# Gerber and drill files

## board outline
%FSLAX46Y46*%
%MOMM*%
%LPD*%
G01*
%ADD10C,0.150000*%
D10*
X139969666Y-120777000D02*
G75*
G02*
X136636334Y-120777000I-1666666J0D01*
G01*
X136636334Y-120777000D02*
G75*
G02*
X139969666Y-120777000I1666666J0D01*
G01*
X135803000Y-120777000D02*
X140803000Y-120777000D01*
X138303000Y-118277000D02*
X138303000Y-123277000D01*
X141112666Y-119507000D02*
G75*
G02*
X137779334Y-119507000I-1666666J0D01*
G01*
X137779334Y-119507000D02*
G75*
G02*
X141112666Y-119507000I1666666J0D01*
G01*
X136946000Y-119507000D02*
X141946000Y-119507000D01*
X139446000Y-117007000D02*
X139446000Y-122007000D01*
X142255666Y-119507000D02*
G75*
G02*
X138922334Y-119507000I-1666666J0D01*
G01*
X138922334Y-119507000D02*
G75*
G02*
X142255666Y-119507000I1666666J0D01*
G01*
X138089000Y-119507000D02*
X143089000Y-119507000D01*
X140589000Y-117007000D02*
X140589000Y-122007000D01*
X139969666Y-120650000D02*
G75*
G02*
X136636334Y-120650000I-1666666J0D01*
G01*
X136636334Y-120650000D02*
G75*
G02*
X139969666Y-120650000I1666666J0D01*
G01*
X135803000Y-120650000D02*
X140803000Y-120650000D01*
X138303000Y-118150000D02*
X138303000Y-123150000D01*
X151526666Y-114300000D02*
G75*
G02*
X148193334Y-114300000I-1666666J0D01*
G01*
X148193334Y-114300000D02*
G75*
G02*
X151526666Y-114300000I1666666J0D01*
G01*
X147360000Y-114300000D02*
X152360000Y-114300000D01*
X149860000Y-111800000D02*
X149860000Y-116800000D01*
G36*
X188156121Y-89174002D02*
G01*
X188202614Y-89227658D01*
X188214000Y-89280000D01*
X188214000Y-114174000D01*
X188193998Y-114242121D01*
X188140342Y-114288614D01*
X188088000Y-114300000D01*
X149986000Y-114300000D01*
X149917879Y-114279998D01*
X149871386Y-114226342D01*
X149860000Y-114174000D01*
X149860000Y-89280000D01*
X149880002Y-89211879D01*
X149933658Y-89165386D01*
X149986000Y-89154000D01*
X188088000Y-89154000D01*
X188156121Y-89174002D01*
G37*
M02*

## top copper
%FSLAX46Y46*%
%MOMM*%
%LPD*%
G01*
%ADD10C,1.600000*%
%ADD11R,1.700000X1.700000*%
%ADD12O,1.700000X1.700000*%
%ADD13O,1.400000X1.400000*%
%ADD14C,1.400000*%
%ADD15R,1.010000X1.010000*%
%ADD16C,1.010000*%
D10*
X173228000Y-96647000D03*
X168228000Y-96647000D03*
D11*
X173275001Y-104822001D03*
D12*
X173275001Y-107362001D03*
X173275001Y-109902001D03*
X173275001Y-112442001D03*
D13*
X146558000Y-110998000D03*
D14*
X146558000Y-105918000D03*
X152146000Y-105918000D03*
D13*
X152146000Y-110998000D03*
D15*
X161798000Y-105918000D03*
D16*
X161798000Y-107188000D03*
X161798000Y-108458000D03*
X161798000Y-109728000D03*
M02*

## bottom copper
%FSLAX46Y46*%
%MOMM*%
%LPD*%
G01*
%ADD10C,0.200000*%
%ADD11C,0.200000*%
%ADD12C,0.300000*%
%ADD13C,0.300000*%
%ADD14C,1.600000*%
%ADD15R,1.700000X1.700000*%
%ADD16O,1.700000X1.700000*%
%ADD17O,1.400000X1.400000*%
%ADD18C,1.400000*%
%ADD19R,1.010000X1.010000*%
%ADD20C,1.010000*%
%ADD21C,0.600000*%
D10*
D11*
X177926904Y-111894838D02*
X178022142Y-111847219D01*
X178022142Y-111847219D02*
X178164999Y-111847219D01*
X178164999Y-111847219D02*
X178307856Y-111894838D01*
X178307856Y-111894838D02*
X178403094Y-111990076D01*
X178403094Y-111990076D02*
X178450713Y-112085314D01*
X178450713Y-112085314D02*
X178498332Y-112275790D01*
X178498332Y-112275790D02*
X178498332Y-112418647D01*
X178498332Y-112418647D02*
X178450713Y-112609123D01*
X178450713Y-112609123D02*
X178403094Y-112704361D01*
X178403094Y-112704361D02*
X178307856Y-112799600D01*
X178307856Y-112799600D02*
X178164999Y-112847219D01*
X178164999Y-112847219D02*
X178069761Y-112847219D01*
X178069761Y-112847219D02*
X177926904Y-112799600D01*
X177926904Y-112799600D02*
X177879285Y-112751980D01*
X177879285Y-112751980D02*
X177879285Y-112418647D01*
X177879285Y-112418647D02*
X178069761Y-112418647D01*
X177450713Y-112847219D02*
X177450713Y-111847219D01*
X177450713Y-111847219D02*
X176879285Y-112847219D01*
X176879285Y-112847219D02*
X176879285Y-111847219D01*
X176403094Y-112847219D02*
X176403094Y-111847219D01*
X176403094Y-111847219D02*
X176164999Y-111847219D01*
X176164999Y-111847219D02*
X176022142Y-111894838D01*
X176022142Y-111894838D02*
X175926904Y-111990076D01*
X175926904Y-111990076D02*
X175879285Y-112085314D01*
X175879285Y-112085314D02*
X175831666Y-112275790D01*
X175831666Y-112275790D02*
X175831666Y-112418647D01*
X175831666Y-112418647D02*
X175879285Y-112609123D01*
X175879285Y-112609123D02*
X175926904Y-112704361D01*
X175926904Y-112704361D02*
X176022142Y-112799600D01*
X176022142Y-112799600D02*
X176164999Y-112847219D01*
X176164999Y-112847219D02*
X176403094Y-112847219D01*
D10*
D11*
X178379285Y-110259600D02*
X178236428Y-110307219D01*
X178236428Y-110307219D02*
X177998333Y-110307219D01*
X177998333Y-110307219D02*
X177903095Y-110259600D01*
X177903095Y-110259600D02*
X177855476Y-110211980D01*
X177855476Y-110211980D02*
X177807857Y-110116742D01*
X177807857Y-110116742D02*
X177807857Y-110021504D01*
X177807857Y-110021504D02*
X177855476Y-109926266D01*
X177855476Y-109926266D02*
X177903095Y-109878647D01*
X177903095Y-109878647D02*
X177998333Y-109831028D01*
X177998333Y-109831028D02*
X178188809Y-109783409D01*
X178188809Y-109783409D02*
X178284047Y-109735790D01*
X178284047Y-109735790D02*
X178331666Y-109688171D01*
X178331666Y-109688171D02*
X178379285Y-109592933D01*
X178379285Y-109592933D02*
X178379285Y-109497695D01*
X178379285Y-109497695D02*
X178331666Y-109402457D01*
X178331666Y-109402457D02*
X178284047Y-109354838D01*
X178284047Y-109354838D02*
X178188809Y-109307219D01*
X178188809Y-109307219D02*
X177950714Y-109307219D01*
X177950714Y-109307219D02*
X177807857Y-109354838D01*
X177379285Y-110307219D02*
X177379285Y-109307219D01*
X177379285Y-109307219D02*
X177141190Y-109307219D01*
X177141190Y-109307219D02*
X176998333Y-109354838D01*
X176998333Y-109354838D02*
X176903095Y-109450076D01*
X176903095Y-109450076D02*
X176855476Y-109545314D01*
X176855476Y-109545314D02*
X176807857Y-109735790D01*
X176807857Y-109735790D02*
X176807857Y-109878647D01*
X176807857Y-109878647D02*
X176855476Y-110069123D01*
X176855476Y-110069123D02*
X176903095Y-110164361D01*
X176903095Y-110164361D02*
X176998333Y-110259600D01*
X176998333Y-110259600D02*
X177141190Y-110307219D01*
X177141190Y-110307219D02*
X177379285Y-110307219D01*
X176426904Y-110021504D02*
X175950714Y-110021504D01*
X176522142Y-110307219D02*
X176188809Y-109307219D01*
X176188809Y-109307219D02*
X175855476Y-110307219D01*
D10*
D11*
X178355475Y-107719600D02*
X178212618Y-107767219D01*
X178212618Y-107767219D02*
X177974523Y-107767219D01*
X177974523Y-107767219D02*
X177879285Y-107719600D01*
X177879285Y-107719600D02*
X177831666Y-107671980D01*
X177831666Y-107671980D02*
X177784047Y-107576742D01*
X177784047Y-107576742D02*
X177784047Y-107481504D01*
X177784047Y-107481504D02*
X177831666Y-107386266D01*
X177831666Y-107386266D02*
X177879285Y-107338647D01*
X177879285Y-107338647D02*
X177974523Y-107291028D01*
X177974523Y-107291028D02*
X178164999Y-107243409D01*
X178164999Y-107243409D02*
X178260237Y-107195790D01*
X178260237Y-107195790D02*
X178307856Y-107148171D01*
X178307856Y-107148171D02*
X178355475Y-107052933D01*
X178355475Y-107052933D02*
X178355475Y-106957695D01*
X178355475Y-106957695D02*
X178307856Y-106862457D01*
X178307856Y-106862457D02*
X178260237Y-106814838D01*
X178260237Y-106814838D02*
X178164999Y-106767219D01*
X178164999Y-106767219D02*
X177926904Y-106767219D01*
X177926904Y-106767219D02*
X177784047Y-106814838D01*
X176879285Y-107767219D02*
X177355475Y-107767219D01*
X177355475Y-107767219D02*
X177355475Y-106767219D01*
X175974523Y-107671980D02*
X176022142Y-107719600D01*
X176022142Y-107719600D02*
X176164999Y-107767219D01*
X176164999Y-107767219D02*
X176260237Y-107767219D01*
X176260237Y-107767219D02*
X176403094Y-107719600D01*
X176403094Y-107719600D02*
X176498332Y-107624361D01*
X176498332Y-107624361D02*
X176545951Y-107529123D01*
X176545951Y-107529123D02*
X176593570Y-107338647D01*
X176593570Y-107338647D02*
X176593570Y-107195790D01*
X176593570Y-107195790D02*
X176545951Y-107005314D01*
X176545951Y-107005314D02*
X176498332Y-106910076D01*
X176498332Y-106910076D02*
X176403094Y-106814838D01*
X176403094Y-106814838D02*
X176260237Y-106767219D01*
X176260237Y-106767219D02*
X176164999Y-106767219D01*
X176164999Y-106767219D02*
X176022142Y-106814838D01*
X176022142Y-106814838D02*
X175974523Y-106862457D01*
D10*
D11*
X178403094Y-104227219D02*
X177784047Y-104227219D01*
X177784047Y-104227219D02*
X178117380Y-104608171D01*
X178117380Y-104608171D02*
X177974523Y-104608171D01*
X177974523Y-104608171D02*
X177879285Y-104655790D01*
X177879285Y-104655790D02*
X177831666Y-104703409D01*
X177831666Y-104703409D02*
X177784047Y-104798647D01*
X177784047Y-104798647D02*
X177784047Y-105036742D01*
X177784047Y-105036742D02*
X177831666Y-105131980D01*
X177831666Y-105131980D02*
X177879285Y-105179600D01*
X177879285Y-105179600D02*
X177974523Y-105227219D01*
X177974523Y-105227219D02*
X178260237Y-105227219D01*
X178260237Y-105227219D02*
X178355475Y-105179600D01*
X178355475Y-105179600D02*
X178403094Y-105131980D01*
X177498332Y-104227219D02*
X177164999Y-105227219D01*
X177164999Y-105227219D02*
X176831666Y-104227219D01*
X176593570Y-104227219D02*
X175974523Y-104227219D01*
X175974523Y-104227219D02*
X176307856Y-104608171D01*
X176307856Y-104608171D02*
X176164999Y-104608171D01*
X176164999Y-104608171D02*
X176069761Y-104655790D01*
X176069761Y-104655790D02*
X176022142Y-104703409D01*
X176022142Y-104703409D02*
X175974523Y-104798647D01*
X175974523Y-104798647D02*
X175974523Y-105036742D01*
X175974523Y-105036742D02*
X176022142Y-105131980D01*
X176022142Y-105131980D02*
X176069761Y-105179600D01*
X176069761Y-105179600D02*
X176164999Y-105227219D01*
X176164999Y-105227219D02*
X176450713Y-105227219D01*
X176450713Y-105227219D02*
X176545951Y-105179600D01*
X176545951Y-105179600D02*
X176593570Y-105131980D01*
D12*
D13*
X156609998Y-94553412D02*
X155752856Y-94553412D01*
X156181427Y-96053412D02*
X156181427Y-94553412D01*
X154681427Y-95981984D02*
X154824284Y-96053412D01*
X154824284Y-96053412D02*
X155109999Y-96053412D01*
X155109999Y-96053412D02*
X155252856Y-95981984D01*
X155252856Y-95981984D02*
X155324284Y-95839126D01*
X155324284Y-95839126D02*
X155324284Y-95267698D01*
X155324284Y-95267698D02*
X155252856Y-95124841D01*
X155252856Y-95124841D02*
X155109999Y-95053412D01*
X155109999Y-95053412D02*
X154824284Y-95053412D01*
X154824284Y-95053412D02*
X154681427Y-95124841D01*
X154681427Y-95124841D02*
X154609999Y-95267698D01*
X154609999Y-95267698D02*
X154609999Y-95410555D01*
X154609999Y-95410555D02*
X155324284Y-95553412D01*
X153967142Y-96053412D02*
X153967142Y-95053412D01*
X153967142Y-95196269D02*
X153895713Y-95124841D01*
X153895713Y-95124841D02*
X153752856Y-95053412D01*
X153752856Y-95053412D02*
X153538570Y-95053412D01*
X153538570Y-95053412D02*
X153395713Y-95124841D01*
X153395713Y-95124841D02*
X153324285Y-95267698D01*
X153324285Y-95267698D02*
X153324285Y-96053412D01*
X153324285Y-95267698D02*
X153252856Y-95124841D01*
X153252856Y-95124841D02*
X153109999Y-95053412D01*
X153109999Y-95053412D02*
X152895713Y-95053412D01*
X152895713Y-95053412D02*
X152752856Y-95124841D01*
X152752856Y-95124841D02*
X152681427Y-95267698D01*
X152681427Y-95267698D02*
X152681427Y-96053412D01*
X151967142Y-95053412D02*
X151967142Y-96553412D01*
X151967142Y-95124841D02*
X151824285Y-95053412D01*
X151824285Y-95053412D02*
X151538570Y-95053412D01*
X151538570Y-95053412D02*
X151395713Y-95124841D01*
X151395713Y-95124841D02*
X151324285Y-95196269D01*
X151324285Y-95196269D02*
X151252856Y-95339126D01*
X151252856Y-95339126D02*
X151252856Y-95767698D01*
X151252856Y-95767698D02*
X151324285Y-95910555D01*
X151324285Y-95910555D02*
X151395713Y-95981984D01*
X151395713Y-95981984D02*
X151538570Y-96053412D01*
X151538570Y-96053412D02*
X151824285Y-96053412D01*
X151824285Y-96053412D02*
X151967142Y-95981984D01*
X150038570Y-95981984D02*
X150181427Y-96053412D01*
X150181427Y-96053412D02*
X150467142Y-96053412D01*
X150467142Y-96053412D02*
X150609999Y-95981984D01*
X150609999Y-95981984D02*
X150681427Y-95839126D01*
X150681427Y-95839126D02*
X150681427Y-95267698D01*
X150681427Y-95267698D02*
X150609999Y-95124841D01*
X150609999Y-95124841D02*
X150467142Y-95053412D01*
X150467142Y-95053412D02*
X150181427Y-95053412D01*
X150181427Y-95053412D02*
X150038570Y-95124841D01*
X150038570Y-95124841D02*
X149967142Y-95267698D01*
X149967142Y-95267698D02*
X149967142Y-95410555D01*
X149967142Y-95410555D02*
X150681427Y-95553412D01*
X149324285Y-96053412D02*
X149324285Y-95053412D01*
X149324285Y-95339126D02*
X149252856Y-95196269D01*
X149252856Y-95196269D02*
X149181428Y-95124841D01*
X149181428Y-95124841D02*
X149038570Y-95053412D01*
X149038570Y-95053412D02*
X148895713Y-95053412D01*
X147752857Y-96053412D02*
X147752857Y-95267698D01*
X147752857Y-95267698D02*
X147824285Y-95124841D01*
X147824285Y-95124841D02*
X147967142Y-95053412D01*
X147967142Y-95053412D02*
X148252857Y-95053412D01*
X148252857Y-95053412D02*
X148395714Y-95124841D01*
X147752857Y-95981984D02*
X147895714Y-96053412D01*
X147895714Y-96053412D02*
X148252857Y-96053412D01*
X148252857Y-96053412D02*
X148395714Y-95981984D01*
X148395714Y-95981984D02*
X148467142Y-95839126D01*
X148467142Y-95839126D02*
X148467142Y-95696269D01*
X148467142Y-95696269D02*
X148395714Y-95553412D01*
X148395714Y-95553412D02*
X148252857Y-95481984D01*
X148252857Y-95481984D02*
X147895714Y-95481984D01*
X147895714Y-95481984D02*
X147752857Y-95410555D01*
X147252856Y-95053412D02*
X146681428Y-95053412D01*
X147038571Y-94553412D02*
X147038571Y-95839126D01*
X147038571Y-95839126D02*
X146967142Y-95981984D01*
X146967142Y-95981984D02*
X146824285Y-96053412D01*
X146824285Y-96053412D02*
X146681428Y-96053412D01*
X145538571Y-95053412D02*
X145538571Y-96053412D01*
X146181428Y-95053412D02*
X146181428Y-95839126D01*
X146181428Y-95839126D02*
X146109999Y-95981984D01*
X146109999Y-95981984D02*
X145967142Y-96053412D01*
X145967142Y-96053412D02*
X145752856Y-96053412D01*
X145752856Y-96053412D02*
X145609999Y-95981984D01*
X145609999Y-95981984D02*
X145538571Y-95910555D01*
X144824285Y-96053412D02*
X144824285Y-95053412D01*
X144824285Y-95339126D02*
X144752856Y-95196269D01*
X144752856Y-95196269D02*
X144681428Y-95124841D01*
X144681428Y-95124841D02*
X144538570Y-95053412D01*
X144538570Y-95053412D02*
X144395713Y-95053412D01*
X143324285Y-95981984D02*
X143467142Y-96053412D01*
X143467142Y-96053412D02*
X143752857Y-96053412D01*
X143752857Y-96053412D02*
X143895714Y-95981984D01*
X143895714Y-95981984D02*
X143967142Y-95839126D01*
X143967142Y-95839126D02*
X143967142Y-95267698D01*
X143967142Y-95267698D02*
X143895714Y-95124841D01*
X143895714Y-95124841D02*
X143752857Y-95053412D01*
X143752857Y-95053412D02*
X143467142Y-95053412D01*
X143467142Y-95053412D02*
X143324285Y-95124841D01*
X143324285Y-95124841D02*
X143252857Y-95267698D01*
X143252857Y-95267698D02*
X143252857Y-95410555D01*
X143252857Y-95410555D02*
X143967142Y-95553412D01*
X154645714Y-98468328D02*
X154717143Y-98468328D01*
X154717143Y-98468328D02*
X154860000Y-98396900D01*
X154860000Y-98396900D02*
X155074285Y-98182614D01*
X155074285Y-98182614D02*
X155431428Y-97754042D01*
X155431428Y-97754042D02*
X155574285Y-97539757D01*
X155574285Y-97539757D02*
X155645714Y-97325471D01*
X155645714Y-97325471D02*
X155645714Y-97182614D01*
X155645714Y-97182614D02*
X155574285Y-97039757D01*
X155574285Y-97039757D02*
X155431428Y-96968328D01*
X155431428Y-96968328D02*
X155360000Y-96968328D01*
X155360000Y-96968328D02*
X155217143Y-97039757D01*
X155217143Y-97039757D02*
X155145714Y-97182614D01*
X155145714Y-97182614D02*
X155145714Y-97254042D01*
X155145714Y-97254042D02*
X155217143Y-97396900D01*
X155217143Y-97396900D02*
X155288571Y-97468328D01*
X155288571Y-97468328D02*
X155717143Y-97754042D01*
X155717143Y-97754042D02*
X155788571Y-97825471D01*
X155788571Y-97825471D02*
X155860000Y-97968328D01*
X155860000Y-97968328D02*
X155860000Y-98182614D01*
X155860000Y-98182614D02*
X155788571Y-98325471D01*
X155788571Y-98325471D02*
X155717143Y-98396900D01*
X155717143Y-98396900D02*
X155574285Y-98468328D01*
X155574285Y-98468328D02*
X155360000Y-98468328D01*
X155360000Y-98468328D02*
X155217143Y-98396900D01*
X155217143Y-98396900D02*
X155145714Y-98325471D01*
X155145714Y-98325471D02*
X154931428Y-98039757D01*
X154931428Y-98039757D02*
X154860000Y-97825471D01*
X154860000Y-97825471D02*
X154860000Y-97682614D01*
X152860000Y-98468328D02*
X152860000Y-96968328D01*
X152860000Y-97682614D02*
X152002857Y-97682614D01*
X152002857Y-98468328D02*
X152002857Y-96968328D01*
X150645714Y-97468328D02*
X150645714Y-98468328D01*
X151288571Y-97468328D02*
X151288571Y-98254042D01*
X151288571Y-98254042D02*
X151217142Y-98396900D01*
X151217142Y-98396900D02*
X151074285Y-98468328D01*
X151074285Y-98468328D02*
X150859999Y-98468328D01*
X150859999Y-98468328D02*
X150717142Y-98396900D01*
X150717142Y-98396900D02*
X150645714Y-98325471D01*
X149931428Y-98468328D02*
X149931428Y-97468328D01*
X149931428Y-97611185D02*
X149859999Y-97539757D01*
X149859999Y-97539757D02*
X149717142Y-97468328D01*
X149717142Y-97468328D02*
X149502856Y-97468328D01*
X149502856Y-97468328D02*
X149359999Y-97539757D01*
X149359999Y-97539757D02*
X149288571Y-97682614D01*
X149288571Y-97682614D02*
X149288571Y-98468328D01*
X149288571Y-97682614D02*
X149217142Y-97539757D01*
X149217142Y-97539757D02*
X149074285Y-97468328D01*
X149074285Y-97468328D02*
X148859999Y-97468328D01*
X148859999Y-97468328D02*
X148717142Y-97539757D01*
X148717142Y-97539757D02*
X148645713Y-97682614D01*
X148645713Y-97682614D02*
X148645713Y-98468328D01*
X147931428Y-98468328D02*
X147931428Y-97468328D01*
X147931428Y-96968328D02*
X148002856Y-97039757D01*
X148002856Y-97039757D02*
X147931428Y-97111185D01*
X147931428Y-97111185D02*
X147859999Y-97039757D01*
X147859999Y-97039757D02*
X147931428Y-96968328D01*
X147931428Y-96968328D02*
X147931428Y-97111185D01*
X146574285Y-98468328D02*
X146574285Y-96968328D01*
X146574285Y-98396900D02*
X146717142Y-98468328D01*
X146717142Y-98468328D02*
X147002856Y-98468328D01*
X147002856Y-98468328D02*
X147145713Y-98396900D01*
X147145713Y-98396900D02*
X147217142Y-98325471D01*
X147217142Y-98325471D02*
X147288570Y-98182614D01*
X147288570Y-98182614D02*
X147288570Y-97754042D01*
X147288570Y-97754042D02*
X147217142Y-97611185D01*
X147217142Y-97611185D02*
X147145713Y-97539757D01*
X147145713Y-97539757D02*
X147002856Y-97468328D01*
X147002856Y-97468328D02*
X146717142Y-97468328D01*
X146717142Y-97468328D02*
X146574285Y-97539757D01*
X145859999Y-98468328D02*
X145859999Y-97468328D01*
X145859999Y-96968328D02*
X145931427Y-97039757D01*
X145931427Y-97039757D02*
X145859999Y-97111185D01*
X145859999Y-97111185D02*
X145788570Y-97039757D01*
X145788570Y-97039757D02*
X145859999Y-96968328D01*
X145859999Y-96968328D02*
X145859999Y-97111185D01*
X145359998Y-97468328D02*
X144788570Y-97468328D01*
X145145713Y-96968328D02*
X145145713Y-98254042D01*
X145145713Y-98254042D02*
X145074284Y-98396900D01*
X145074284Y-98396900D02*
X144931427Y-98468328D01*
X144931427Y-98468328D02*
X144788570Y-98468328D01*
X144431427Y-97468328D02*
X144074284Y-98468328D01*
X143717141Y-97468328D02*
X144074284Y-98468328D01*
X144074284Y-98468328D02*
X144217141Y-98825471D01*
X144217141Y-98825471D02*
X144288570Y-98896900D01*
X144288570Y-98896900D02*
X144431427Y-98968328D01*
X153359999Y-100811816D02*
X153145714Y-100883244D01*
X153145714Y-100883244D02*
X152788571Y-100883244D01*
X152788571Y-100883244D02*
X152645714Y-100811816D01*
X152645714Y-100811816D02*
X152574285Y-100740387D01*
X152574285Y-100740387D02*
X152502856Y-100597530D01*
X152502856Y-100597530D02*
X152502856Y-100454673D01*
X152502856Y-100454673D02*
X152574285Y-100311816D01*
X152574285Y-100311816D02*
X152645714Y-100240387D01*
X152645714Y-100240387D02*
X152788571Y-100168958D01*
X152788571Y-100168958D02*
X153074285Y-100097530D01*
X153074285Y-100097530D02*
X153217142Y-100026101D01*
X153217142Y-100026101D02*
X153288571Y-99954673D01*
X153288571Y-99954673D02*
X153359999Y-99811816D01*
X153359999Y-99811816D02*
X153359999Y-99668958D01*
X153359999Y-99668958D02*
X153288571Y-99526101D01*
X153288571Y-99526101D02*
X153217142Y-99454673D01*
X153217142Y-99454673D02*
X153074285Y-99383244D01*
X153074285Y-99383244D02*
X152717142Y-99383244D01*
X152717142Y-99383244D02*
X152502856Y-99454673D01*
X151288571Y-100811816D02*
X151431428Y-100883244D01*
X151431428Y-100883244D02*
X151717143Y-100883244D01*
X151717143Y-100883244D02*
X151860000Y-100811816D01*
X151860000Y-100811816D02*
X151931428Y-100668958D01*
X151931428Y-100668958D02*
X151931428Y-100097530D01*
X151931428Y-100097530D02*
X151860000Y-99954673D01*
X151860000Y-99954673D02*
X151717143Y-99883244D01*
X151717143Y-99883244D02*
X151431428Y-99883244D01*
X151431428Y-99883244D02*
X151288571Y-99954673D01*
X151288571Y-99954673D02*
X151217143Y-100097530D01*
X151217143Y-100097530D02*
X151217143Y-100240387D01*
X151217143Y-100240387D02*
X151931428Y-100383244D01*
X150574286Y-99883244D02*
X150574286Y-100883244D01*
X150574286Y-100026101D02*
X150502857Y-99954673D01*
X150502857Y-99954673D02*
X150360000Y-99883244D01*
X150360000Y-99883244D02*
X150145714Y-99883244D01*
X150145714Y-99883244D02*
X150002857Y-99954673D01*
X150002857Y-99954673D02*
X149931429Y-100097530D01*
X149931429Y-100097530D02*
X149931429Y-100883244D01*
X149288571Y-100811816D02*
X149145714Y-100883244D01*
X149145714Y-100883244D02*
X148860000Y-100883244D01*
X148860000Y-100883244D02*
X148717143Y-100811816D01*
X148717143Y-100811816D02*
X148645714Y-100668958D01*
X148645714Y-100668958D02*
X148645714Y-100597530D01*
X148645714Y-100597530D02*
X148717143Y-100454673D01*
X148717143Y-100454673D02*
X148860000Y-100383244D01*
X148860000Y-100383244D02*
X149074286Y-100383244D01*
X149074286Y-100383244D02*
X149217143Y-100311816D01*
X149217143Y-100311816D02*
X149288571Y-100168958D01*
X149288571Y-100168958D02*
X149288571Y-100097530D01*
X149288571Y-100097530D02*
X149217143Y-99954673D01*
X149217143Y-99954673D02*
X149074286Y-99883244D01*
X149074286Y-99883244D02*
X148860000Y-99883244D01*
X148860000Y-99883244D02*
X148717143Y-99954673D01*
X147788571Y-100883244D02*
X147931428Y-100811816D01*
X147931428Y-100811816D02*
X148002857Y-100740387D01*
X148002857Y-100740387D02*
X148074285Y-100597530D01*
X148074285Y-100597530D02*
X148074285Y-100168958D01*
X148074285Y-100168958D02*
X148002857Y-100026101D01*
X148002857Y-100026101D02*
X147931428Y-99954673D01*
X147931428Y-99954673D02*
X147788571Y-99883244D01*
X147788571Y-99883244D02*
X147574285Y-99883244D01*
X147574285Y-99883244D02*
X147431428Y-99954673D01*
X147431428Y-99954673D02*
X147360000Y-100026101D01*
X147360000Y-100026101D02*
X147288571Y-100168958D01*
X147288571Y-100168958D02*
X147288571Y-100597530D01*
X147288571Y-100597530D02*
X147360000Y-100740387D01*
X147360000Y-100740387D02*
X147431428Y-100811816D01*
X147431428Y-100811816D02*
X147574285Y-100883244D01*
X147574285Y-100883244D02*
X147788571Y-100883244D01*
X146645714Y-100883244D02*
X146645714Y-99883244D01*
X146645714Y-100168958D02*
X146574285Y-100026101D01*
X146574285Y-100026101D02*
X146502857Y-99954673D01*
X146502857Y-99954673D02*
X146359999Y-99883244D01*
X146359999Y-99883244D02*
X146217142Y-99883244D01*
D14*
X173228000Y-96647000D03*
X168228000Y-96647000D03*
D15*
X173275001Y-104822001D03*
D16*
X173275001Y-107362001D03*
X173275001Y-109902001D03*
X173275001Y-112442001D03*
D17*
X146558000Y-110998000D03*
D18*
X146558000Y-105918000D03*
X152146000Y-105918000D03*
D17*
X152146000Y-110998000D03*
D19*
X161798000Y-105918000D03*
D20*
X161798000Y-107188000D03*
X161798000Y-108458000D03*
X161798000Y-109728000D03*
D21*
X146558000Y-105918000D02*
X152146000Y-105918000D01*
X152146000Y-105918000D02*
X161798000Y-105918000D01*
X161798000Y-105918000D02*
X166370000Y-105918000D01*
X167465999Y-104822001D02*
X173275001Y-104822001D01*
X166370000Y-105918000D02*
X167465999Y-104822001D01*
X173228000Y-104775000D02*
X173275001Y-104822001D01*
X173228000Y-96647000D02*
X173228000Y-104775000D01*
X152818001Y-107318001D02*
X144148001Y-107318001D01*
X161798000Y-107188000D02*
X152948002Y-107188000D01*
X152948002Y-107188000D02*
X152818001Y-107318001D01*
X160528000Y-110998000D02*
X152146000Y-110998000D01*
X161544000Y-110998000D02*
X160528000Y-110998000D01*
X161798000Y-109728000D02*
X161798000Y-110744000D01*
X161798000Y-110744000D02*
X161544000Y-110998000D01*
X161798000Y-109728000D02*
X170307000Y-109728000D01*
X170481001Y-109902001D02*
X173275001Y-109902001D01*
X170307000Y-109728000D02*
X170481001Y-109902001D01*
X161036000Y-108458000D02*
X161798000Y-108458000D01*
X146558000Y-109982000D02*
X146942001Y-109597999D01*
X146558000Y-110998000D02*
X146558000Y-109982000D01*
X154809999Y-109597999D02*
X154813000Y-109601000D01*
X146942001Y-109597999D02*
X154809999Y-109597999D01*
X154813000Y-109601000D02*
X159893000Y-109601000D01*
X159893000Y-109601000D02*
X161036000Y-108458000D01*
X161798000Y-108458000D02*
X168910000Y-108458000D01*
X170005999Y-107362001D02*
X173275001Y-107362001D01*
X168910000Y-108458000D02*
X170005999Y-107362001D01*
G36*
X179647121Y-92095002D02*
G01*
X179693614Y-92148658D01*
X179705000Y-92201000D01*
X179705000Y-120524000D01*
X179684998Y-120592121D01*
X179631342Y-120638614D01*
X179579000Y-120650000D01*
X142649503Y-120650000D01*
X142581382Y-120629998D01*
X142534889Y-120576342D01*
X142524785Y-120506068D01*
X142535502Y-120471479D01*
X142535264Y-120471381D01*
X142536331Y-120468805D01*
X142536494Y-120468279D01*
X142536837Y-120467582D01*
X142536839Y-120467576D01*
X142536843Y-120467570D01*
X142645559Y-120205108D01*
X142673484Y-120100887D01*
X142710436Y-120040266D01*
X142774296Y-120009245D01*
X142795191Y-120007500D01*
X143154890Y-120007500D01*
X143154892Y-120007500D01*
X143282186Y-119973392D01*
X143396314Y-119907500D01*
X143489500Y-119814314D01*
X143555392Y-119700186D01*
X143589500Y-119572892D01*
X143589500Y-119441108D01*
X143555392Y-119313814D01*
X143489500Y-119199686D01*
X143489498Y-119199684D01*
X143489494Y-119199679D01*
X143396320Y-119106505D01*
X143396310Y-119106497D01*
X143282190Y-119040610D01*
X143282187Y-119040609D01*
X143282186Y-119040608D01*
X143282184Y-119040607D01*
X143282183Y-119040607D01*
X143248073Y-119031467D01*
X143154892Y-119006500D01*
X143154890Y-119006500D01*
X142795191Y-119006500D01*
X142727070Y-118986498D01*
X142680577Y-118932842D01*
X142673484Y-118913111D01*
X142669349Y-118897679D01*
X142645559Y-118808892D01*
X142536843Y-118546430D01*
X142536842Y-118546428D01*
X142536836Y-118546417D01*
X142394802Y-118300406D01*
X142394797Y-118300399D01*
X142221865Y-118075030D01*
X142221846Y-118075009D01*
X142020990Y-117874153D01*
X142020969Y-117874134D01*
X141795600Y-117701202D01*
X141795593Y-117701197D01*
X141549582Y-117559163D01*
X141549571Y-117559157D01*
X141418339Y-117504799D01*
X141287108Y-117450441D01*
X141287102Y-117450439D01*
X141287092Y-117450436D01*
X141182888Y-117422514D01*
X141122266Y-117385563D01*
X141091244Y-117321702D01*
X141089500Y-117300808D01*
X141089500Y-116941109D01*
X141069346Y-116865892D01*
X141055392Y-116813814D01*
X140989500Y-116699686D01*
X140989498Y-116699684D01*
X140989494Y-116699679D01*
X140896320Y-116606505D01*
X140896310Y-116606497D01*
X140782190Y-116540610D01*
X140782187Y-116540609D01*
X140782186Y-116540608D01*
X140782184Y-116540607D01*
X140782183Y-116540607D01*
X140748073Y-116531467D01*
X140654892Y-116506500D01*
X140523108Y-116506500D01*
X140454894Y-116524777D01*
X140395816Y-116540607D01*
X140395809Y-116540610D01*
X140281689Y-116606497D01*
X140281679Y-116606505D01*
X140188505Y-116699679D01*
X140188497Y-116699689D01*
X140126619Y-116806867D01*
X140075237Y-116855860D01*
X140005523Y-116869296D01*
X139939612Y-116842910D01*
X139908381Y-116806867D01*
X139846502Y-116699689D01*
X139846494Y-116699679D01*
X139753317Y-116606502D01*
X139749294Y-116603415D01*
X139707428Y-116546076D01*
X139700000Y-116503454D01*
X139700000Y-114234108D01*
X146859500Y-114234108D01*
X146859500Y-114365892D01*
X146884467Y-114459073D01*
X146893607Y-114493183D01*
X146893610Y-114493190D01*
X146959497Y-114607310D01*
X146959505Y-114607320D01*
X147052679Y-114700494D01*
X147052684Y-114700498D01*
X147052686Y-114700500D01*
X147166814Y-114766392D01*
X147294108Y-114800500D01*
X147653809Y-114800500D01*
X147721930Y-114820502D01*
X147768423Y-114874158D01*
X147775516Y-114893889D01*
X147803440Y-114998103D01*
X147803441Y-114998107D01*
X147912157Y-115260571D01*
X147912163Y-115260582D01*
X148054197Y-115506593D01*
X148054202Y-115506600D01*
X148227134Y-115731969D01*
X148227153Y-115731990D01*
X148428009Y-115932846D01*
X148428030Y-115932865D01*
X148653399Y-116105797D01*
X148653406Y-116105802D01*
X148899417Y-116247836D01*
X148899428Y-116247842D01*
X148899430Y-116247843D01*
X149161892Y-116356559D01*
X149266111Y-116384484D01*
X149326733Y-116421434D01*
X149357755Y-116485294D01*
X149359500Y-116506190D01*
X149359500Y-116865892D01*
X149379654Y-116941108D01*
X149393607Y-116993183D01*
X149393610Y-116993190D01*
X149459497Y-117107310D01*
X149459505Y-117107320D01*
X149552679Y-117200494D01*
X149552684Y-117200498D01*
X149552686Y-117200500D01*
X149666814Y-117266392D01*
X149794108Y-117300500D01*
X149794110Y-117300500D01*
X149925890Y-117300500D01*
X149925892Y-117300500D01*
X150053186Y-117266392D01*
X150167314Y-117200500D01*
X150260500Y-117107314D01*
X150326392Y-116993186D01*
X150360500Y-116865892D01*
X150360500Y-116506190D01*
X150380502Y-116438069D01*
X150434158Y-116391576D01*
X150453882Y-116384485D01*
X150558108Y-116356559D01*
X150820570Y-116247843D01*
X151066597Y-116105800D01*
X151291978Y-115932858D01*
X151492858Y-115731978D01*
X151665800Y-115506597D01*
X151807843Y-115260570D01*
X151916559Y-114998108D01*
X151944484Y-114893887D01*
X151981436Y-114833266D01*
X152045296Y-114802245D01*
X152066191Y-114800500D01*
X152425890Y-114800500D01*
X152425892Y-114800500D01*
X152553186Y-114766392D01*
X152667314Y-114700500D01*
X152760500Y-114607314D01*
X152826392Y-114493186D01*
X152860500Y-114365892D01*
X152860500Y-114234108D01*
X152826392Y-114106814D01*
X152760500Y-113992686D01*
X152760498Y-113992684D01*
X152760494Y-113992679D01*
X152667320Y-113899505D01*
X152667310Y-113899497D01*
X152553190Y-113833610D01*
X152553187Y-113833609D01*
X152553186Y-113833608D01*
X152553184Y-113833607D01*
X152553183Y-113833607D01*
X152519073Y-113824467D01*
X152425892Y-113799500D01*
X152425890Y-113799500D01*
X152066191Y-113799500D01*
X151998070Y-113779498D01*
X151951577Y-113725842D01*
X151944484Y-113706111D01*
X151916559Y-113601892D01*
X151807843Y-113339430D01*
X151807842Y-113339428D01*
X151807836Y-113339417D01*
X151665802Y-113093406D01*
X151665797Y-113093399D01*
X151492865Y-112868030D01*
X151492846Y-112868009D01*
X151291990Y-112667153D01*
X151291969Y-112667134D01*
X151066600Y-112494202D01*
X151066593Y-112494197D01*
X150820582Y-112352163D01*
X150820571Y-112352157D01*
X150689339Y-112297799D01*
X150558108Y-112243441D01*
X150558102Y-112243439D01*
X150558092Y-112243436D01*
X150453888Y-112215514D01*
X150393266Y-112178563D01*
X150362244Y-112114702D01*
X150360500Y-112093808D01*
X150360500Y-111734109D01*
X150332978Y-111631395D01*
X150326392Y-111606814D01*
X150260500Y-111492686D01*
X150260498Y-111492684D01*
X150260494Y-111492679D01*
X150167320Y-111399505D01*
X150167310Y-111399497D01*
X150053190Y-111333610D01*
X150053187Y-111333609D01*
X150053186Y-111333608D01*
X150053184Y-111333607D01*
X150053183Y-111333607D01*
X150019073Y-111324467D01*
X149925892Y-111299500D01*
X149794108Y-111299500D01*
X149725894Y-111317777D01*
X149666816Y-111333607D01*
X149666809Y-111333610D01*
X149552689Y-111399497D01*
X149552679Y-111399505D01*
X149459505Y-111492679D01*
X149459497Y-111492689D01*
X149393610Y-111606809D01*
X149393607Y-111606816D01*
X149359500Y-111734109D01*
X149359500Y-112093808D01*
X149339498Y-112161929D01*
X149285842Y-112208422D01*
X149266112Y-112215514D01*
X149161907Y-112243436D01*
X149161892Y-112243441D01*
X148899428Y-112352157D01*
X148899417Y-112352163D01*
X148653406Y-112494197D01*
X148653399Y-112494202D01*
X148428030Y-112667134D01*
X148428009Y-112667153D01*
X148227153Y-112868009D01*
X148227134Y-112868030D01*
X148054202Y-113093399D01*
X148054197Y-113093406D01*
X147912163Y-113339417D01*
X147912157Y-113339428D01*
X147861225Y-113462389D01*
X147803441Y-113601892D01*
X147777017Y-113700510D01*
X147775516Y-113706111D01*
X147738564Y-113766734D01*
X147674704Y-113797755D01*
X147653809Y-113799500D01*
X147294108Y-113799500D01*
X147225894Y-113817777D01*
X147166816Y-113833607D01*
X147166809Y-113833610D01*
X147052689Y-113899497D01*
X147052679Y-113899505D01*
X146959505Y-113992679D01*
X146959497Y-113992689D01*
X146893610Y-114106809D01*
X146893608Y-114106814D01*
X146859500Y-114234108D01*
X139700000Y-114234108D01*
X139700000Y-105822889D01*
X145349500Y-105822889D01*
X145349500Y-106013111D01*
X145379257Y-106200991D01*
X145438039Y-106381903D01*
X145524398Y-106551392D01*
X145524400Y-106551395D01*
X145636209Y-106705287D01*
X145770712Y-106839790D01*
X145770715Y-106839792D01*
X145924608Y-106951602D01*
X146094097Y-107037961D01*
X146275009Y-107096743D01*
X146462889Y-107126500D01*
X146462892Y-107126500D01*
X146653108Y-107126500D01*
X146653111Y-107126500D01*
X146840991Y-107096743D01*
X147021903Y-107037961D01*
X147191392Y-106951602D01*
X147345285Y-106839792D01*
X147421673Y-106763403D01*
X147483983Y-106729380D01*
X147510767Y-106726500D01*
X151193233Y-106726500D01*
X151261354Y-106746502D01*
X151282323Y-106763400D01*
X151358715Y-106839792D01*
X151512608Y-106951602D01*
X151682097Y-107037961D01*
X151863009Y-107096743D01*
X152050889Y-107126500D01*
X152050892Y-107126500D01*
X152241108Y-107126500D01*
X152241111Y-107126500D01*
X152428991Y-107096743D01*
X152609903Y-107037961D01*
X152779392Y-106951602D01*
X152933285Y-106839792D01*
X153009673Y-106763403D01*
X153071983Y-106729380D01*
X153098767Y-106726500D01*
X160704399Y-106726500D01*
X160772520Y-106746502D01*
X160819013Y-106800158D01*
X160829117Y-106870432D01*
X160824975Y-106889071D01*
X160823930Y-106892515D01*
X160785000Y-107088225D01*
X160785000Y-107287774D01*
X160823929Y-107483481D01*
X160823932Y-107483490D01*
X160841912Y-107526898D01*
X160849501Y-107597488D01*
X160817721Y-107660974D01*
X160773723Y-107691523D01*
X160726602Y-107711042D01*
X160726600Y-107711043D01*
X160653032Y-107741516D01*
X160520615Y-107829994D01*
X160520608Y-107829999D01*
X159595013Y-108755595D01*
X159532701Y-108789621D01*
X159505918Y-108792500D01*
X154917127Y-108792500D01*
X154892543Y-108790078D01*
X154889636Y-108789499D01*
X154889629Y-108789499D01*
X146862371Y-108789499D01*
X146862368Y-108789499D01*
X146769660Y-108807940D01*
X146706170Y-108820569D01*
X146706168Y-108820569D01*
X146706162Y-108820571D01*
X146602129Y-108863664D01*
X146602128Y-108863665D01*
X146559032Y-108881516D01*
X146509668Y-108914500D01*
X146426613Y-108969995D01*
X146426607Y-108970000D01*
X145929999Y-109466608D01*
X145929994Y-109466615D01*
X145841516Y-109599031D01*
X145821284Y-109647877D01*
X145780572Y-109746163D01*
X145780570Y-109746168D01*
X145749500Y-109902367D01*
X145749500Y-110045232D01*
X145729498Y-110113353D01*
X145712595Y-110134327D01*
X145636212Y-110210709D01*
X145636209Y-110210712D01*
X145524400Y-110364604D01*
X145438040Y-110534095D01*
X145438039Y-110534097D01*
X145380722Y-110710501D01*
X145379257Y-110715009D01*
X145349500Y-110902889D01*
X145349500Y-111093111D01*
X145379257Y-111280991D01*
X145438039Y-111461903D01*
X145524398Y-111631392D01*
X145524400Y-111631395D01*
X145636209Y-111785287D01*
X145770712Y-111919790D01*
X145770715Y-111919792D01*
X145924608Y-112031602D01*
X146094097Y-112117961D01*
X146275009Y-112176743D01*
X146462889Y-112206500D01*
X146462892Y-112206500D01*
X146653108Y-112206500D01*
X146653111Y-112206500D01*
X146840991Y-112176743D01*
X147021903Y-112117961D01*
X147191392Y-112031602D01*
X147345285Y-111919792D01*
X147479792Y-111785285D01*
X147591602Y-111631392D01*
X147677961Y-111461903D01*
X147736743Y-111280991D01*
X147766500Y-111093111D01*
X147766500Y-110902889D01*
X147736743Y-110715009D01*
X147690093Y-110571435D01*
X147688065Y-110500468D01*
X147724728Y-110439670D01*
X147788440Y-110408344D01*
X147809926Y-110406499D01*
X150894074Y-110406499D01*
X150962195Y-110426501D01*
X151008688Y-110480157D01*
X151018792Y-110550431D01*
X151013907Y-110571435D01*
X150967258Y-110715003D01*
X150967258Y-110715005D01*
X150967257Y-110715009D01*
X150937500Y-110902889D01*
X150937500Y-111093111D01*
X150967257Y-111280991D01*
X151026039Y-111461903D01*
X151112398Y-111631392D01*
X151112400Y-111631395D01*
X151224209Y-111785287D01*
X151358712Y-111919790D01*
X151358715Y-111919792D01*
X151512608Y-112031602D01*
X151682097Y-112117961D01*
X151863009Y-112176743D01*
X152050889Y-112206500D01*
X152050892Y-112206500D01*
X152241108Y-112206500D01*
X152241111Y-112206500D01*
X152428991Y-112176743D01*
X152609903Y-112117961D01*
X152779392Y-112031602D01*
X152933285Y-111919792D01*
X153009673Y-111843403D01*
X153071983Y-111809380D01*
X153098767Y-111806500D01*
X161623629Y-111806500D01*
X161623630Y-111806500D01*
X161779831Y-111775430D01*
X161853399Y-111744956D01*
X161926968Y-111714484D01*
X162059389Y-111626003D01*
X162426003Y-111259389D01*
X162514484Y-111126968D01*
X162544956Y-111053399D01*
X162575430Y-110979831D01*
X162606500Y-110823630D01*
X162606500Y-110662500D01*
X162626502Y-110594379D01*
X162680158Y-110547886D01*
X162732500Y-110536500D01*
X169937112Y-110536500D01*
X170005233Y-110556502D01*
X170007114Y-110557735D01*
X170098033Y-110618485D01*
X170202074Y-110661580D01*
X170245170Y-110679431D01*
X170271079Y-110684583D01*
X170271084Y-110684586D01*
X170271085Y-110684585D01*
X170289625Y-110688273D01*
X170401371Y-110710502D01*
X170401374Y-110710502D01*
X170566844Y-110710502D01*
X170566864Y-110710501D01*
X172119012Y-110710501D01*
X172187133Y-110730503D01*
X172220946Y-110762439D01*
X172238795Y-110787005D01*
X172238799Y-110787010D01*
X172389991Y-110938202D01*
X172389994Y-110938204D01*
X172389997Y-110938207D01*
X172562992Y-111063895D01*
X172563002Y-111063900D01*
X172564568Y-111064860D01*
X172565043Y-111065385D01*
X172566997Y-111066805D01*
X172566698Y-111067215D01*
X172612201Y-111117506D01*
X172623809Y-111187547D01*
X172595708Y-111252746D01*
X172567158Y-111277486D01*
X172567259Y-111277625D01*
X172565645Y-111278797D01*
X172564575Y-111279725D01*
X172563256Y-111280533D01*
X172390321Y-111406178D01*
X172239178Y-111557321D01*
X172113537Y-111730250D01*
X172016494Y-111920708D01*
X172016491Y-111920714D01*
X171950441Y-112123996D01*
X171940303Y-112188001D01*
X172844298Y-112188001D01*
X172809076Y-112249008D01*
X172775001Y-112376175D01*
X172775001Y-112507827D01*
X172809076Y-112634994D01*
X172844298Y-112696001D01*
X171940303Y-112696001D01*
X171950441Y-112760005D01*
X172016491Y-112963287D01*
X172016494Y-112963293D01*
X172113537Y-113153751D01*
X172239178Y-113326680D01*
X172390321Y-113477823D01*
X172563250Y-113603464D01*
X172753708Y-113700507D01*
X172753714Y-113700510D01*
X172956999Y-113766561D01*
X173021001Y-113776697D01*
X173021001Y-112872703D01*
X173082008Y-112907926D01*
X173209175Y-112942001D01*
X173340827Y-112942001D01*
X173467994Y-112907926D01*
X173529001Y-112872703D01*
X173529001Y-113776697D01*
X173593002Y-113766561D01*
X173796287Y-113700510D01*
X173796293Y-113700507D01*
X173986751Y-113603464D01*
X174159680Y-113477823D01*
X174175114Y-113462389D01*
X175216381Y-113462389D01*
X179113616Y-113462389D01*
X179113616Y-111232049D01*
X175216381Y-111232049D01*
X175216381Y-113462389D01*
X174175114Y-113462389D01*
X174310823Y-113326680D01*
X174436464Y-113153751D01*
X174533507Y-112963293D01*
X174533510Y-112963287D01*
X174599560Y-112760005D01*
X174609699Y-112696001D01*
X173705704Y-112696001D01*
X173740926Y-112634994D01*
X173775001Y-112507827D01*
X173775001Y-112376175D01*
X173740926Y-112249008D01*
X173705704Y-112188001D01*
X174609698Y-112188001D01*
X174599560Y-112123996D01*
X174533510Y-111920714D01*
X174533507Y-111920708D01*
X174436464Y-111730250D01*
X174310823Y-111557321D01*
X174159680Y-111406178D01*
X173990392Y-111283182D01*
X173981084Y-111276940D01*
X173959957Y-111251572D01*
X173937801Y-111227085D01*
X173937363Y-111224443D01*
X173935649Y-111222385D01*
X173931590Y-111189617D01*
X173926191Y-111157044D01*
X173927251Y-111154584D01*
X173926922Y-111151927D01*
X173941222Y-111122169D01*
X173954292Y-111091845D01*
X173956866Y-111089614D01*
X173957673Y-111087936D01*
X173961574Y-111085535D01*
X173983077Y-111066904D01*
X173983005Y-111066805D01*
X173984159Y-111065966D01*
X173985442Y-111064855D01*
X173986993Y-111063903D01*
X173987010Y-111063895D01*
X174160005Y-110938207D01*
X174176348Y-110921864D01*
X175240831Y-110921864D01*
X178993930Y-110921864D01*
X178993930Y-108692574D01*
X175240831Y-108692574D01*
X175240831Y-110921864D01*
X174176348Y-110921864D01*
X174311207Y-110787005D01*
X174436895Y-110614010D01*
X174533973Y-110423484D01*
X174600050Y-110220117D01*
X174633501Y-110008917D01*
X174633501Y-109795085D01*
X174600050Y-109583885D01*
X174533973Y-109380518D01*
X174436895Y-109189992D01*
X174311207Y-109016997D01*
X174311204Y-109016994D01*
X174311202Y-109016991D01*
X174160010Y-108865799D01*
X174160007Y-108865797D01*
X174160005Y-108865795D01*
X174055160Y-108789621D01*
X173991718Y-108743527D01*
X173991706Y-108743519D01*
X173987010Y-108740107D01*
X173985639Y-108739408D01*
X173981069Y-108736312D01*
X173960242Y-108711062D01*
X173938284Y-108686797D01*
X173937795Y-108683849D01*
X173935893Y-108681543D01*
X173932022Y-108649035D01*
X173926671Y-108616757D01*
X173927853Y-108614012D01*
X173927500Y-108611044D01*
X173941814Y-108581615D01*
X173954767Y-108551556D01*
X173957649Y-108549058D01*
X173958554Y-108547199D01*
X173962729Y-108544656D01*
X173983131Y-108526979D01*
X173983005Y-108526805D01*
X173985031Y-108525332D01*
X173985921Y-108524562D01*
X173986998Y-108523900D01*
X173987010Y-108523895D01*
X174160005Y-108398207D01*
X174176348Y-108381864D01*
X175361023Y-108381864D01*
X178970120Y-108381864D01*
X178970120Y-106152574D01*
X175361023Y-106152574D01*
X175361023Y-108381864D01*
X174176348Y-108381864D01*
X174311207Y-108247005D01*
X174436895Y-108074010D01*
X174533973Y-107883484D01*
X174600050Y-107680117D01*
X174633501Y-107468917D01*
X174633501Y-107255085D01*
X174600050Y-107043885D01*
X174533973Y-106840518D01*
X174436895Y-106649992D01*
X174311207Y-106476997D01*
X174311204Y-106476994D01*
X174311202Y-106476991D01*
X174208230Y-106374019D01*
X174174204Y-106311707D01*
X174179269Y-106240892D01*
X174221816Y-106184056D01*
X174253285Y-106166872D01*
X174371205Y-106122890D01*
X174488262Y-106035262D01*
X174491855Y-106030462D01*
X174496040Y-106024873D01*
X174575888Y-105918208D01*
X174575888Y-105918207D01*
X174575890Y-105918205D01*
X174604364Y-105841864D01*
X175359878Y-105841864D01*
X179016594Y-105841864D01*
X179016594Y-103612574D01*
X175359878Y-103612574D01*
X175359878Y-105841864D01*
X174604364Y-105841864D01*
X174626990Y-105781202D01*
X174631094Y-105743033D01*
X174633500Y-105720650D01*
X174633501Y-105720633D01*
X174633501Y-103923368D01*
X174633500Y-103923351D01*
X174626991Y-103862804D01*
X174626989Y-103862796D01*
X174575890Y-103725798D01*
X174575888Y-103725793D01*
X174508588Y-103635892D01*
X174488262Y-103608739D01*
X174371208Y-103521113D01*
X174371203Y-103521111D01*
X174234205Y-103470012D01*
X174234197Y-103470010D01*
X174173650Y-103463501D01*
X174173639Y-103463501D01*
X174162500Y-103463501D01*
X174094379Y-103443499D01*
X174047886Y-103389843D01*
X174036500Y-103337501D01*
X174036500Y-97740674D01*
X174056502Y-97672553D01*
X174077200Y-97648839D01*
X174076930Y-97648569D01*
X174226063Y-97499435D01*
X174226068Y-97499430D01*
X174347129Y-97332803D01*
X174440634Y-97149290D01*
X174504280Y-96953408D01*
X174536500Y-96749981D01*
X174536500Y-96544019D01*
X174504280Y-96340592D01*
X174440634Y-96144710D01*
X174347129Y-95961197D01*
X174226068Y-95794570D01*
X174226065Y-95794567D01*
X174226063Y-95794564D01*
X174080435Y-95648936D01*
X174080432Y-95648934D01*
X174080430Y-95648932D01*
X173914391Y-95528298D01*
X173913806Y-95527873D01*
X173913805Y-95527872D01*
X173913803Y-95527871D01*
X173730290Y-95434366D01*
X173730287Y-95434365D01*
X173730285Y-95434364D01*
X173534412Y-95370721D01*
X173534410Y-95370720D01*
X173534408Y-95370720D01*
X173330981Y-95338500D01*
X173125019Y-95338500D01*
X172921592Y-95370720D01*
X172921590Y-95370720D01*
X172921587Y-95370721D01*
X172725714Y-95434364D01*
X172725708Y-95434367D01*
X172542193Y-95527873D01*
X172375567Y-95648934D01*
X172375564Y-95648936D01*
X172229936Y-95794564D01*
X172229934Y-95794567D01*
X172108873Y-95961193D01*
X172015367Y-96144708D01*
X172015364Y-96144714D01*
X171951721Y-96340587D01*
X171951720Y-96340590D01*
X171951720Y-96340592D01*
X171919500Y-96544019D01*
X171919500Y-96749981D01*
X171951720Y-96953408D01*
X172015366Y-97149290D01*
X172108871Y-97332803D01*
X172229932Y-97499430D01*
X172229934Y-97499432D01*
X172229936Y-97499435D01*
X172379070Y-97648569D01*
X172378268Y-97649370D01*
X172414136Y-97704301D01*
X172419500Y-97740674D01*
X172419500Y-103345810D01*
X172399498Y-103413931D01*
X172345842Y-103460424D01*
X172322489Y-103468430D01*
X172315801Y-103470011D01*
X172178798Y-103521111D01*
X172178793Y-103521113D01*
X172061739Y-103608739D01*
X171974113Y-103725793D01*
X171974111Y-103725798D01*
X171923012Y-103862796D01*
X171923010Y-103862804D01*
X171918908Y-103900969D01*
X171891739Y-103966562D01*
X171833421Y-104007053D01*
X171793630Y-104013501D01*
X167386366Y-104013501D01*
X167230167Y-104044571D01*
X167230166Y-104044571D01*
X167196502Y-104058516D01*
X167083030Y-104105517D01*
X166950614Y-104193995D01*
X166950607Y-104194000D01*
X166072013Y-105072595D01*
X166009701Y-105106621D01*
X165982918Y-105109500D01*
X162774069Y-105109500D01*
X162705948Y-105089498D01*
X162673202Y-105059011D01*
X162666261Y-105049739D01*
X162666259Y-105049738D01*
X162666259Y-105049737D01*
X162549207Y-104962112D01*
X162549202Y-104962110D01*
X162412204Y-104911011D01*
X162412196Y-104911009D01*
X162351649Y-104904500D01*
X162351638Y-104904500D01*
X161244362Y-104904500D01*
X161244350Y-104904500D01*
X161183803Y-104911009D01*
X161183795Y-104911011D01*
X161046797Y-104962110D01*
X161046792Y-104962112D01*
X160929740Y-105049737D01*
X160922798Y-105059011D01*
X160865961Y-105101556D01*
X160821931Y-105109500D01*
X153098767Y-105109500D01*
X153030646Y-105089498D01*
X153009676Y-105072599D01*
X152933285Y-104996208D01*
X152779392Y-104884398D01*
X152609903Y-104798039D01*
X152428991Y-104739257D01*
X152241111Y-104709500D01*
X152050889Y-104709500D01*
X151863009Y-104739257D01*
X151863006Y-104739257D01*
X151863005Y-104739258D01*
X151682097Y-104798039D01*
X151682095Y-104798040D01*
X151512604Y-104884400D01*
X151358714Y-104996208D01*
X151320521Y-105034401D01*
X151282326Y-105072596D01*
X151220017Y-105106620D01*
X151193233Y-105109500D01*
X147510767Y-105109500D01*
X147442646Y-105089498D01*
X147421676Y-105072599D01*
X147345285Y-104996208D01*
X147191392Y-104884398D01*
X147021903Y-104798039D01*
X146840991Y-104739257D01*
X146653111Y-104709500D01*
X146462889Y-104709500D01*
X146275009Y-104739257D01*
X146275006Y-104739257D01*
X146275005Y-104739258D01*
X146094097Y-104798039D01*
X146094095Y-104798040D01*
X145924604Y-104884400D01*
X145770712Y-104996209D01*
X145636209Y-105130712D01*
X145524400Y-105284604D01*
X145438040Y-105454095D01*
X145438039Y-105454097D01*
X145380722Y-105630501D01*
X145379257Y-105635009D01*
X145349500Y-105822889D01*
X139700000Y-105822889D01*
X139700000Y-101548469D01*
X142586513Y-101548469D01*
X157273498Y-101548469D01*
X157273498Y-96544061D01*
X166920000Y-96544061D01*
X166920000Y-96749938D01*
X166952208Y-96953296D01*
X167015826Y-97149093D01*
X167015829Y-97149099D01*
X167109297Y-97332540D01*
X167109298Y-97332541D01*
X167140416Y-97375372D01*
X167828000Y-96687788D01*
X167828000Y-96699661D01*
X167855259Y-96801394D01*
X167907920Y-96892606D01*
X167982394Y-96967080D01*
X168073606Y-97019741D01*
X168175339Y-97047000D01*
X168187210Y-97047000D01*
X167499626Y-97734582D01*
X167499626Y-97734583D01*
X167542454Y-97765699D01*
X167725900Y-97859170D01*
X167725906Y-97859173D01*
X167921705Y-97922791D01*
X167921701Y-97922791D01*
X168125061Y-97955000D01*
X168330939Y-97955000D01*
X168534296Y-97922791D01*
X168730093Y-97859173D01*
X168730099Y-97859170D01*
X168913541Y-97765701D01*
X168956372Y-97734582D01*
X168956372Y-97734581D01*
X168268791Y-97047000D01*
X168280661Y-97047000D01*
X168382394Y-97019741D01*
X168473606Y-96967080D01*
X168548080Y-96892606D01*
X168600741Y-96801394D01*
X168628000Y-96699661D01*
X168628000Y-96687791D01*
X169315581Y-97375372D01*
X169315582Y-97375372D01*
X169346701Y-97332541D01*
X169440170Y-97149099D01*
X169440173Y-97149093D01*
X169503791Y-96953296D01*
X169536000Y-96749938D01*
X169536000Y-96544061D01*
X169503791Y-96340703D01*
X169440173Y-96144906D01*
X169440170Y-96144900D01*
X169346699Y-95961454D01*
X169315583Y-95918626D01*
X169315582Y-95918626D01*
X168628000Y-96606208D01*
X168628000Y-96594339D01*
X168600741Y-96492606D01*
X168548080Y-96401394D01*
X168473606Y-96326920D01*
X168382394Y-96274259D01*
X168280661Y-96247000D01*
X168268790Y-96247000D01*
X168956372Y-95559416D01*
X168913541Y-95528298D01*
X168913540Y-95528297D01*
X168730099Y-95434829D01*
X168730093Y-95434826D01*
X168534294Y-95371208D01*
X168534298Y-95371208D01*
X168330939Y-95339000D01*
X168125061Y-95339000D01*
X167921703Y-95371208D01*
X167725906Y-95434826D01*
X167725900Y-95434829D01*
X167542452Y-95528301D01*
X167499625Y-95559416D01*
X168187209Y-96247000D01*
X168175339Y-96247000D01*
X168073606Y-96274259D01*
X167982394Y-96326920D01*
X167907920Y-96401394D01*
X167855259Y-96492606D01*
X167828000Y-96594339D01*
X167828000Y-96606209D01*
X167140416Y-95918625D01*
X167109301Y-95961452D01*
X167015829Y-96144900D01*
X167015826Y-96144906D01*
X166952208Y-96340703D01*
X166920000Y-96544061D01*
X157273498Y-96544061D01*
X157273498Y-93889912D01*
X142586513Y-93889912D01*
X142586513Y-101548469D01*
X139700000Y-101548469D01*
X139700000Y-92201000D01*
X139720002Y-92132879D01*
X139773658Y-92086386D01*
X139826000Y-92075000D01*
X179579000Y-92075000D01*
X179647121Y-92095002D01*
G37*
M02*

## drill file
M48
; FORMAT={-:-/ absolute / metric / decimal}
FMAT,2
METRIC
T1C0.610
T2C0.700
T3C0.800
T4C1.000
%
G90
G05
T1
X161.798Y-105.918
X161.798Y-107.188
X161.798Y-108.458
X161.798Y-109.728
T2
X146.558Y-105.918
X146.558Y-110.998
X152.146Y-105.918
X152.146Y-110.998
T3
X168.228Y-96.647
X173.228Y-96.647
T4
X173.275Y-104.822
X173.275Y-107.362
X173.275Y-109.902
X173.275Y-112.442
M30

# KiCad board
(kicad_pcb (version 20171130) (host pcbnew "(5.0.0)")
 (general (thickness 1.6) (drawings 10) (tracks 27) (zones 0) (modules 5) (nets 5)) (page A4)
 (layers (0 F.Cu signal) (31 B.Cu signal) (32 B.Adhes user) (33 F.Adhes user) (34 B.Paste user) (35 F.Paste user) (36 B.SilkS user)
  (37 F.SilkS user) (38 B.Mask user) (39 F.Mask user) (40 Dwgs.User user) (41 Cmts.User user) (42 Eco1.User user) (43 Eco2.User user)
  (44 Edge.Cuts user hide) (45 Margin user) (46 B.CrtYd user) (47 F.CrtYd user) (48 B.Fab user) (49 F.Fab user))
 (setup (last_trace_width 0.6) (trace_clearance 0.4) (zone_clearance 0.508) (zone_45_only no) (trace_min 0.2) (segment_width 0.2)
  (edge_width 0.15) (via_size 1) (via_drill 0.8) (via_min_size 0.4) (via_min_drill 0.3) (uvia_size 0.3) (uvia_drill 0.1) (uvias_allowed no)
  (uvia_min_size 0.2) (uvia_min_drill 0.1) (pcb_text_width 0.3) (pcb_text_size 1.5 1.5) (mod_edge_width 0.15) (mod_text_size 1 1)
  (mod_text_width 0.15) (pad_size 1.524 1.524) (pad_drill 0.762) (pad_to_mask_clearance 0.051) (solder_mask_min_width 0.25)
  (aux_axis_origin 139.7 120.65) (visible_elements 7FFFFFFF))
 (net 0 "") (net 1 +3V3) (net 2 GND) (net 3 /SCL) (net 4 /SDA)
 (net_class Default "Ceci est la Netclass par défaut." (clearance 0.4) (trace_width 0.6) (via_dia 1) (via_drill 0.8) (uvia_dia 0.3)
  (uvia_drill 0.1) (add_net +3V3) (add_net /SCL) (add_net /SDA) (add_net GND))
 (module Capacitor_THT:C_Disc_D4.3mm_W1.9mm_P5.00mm (layer F.Cu) (at 173.228 96.647 180)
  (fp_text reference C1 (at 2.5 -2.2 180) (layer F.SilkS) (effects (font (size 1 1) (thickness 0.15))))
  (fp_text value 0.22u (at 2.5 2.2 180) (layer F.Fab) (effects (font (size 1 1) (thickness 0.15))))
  (pad 1 thru_hole circle (at 0 0 180) (size 1.6 1.6) (drill 0.8) (layers *.Cu *.Mask) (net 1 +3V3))
  (pad 2 thru_hole circle (at 5 0 180) (size 1.6 1.6) (drill 0.8) (layers *.Cu *.Mask) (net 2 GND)))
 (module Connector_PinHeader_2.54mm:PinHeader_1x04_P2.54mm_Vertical (layer F.Cu) (at 173.275001 104.822001)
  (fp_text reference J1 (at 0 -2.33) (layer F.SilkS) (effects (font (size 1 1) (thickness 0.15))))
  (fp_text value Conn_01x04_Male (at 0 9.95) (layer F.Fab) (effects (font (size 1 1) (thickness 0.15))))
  (pad 1 thru_hole rect (at 0 0) (size 1.7 1.7) (drill 1) (layers *.Cu *.Mask) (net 1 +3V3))
  (pad 2 thru_hole oval (at 0 2.54) (size 1.7 1.7) (drill 1) (layers *.Cu *.Mask) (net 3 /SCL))
  (pad 3 thru_hole oval (at 0 5.08) (size 1.7 1.7) (drill 1) (layers *.Cu *.Mask) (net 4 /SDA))
  (pad 4 thru_hole oval (at 0 7.62) (size 1.7 1.7) (drill 1) (layers *.Cu *.Mask) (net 2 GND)))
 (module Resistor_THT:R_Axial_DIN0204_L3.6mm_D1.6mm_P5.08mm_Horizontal (layer F.Cu) (at 146.558 105.918 270)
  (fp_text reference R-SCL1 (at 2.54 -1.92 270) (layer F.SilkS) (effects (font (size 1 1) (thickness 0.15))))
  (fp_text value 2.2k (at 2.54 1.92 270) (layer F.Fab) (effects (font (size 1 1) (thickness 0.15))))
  (pad 2 thru_hole oval (at 5.08 0 270) (size 1.4 1.4) (drill 0.7) (layers *.Cu *.Mask) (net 3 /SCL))
  (pad 1 thru_hole circle (at 0 0 270) (size 1.4 1.4) (drill 0.7) (layers *.Cu *.Mask) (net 1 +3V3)))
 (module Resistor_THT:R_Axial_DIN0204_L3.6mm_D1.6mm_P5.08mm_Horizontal (layer F.Cu) (at 152.146 105.918 270)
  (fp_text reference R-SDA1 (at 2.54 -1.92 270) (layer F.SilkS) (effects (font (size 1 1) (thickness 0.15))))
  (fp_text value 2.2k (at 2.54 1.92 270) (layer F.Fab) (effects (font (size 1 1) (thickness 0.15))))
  (pad 1 thru_hole circle (at 0 0 270) (size 1.4 1.4) (drill 0.7) (layers *.Cu *.Mask) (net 1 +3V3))
  (pad 2 thru_hole oval (at 5.08 0 270) (size 1.4 1.4) (drill 0.7) (layers *.Cu *.Mask) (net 4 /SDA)))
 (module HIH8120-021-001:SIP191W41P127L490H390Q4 (layer F.Cu) (at 161.798 107.823 270)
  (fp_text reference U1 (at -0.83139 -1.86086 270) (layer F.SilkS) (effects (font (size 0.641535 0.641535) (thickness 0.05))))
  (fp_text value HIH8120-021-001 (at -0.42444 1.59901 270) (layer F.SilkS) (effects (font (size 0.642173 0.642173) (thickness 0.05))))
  (pad 1 thru_hole rect (at -1.905 0 270) (size 1.01 1.01) (drill 0.61) (layers *.Cu *.Mask) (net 1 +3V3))
  (pad 2 thru_hole circle (at -0.635 0 270) (size 1.01 1.01) (drill 0.61) (layers *.Cu *.Mask) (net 2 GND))
  (pad 3 thru_hole circle (at 0.635 0 270) (size 1.01 1.01) (drill 0.61) (layers *.Cu *.Mask) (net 3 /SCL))
  (pad 4 thru_hole circle (at 1.905 0 270) (size 1.01 1.01) (drill 0.61) (layers *.Cu *.Mask) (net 4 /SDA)))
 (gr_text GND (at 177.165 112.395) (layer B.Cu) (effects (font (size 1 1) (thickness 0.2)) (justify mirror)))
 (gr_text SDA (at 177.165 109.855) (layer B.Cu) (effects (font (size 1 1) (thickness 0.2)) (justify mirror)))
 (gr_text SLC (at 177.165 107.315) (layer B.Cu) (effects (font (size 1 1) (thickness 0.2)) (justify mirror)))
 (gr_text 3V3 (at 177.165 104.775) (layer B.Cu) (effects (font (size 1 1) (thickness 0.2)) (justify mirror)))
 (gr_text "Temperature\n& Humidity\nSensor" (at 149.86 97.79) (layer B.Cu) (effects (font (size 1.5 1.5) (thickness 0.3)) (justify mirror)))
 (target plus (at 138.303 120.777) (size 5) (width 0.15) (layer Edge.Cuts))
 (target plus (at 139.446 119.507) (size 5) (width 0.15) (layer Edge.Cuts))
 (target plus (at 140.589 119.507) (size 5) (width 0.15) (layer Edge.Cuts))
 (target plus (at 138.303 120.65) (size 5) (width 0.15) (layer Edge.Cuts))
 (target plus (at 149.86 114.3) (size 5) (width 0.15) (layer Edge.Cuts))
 (segment (start 146.558 105.918) (end 152.146 105.918) (width 0.6) (layer B.Cu) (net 1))
 (segment (start 152.146 105.918) (end 161.798 105.918) (width 0.6) (layer B.Cu) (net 1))
 (segment (start 161.798 105.918) (end 166.37 105.918) (width 0.6) (layer B.Cu) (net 1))
 (segment (start 167.465999 104.822001) (end 173.275001 104.822001) (width 0.6) (layer B.Cu) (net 1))
 (segment (start 166.37 105.918) (end 167.465999 104.822001) (width 0.6) (layer B.Cu) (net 1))
 (segment (start 173.228 104.775) (end 173.275001 104.822001) (width 0.6) (layer B.Cu) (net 1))
 (segment (start 173.228 96.647) (end 173.228 104.775) (width 0.6) (layer B.Cu) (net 1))
 (segment (start 152.818001 107.318001) (end 144.148001 107.318001) (width 0.6) (layer B.Cu) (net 2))
 (segment (start 161.798 107.188) (end 152.948002 107.188) (width 0.6) (layer B.Cu) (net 2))
 (segment (start 152.948002 107.188) (end 152.818001 107.318001) (width 0.6) (layer B.Cu) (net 2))
 (segment (start 160.528 110.998) (end 152.146 110.998) (width 0.6) (layer B.Cu) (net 4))
 (segment (start 161.544 110.998) (end 160.528 110.998) (width 0.6) (layer B.Cu) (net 4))
 (segment (start 161.798 109.728) (end 161.798 110.744) (width 0.6) (layer B.Cu) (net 4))
 (segment (start 161.798 110.744) (end 161.544 110.998) (width 0.6) (layer B.Cu) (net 4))
 (segment (start 161.798 109.728) (end 170.307 109.728) (width 0.6) (layer B.Cu) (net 4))
 (segment (start 170.481001 109.902001) (end 173.275001 109.902001) (width 0.6) (layer B.Cu) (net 4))
 (segment (start 170.307 109.728) (end 170.481001 109.902001) (width 0.6) (layer B.Cu) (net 4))
 (segment (start 161.036 108.458) (end 161.798 108.458) (width 0.6) (layer B.Cu) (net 3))
 (segment (start 146.558 109.982) (end 146.942001 109.597999) (width 0.6) (layer B.Cu) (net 3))
 (segment (start 146.558 110.998) (end 146.558 109.982) (width 0.6) (layer B.Cu) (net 3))
 (segment (start 154.809999 109.597999) (end 154.813 109.601) (width 0.6) (layer B.Cu) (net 3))
 (segment (start 146.942001 109.597999) (end 154.809999 109.597999) (width 0.6) (layer B.Cu) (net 3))
 (segment (start 154.813 109.601) (end 159.893 109.601) (width 0.6) (layer B.Cu) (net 3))
 (segment (start 159.893 109.601) (end 161.036 108.458) (width 0.6) (layer B.Cu) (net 3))
 (segment (start 161.798 108.458) (end 168.91 108.458) (width 0.6) (layer B.Cu) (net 3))
 (segment (start 170.005999 107.362001) (end 173.275001 107.362001) (width 0.6) (layer B.Cu) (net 3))
 (segment (start 168.91 108.458) (end 170.005999 107.362001) (width 0.6) (layer B.Cu) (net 3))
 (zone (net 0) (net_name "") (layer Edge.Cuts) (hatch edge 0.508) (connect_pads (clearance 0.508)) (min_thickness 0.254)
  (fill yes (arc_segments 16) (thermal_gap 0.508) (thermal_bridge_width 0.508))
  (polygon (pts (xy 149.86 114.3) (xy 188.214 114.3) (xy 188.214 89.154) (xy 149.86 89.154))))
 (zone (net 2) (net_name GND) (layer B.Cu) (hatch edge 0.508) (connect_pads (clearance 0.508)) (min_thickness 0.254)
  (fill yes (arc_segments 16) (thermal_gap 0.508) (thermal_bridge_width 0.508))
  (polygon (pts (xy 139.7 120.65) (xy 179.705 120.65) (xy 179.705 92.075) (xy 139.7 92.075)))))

